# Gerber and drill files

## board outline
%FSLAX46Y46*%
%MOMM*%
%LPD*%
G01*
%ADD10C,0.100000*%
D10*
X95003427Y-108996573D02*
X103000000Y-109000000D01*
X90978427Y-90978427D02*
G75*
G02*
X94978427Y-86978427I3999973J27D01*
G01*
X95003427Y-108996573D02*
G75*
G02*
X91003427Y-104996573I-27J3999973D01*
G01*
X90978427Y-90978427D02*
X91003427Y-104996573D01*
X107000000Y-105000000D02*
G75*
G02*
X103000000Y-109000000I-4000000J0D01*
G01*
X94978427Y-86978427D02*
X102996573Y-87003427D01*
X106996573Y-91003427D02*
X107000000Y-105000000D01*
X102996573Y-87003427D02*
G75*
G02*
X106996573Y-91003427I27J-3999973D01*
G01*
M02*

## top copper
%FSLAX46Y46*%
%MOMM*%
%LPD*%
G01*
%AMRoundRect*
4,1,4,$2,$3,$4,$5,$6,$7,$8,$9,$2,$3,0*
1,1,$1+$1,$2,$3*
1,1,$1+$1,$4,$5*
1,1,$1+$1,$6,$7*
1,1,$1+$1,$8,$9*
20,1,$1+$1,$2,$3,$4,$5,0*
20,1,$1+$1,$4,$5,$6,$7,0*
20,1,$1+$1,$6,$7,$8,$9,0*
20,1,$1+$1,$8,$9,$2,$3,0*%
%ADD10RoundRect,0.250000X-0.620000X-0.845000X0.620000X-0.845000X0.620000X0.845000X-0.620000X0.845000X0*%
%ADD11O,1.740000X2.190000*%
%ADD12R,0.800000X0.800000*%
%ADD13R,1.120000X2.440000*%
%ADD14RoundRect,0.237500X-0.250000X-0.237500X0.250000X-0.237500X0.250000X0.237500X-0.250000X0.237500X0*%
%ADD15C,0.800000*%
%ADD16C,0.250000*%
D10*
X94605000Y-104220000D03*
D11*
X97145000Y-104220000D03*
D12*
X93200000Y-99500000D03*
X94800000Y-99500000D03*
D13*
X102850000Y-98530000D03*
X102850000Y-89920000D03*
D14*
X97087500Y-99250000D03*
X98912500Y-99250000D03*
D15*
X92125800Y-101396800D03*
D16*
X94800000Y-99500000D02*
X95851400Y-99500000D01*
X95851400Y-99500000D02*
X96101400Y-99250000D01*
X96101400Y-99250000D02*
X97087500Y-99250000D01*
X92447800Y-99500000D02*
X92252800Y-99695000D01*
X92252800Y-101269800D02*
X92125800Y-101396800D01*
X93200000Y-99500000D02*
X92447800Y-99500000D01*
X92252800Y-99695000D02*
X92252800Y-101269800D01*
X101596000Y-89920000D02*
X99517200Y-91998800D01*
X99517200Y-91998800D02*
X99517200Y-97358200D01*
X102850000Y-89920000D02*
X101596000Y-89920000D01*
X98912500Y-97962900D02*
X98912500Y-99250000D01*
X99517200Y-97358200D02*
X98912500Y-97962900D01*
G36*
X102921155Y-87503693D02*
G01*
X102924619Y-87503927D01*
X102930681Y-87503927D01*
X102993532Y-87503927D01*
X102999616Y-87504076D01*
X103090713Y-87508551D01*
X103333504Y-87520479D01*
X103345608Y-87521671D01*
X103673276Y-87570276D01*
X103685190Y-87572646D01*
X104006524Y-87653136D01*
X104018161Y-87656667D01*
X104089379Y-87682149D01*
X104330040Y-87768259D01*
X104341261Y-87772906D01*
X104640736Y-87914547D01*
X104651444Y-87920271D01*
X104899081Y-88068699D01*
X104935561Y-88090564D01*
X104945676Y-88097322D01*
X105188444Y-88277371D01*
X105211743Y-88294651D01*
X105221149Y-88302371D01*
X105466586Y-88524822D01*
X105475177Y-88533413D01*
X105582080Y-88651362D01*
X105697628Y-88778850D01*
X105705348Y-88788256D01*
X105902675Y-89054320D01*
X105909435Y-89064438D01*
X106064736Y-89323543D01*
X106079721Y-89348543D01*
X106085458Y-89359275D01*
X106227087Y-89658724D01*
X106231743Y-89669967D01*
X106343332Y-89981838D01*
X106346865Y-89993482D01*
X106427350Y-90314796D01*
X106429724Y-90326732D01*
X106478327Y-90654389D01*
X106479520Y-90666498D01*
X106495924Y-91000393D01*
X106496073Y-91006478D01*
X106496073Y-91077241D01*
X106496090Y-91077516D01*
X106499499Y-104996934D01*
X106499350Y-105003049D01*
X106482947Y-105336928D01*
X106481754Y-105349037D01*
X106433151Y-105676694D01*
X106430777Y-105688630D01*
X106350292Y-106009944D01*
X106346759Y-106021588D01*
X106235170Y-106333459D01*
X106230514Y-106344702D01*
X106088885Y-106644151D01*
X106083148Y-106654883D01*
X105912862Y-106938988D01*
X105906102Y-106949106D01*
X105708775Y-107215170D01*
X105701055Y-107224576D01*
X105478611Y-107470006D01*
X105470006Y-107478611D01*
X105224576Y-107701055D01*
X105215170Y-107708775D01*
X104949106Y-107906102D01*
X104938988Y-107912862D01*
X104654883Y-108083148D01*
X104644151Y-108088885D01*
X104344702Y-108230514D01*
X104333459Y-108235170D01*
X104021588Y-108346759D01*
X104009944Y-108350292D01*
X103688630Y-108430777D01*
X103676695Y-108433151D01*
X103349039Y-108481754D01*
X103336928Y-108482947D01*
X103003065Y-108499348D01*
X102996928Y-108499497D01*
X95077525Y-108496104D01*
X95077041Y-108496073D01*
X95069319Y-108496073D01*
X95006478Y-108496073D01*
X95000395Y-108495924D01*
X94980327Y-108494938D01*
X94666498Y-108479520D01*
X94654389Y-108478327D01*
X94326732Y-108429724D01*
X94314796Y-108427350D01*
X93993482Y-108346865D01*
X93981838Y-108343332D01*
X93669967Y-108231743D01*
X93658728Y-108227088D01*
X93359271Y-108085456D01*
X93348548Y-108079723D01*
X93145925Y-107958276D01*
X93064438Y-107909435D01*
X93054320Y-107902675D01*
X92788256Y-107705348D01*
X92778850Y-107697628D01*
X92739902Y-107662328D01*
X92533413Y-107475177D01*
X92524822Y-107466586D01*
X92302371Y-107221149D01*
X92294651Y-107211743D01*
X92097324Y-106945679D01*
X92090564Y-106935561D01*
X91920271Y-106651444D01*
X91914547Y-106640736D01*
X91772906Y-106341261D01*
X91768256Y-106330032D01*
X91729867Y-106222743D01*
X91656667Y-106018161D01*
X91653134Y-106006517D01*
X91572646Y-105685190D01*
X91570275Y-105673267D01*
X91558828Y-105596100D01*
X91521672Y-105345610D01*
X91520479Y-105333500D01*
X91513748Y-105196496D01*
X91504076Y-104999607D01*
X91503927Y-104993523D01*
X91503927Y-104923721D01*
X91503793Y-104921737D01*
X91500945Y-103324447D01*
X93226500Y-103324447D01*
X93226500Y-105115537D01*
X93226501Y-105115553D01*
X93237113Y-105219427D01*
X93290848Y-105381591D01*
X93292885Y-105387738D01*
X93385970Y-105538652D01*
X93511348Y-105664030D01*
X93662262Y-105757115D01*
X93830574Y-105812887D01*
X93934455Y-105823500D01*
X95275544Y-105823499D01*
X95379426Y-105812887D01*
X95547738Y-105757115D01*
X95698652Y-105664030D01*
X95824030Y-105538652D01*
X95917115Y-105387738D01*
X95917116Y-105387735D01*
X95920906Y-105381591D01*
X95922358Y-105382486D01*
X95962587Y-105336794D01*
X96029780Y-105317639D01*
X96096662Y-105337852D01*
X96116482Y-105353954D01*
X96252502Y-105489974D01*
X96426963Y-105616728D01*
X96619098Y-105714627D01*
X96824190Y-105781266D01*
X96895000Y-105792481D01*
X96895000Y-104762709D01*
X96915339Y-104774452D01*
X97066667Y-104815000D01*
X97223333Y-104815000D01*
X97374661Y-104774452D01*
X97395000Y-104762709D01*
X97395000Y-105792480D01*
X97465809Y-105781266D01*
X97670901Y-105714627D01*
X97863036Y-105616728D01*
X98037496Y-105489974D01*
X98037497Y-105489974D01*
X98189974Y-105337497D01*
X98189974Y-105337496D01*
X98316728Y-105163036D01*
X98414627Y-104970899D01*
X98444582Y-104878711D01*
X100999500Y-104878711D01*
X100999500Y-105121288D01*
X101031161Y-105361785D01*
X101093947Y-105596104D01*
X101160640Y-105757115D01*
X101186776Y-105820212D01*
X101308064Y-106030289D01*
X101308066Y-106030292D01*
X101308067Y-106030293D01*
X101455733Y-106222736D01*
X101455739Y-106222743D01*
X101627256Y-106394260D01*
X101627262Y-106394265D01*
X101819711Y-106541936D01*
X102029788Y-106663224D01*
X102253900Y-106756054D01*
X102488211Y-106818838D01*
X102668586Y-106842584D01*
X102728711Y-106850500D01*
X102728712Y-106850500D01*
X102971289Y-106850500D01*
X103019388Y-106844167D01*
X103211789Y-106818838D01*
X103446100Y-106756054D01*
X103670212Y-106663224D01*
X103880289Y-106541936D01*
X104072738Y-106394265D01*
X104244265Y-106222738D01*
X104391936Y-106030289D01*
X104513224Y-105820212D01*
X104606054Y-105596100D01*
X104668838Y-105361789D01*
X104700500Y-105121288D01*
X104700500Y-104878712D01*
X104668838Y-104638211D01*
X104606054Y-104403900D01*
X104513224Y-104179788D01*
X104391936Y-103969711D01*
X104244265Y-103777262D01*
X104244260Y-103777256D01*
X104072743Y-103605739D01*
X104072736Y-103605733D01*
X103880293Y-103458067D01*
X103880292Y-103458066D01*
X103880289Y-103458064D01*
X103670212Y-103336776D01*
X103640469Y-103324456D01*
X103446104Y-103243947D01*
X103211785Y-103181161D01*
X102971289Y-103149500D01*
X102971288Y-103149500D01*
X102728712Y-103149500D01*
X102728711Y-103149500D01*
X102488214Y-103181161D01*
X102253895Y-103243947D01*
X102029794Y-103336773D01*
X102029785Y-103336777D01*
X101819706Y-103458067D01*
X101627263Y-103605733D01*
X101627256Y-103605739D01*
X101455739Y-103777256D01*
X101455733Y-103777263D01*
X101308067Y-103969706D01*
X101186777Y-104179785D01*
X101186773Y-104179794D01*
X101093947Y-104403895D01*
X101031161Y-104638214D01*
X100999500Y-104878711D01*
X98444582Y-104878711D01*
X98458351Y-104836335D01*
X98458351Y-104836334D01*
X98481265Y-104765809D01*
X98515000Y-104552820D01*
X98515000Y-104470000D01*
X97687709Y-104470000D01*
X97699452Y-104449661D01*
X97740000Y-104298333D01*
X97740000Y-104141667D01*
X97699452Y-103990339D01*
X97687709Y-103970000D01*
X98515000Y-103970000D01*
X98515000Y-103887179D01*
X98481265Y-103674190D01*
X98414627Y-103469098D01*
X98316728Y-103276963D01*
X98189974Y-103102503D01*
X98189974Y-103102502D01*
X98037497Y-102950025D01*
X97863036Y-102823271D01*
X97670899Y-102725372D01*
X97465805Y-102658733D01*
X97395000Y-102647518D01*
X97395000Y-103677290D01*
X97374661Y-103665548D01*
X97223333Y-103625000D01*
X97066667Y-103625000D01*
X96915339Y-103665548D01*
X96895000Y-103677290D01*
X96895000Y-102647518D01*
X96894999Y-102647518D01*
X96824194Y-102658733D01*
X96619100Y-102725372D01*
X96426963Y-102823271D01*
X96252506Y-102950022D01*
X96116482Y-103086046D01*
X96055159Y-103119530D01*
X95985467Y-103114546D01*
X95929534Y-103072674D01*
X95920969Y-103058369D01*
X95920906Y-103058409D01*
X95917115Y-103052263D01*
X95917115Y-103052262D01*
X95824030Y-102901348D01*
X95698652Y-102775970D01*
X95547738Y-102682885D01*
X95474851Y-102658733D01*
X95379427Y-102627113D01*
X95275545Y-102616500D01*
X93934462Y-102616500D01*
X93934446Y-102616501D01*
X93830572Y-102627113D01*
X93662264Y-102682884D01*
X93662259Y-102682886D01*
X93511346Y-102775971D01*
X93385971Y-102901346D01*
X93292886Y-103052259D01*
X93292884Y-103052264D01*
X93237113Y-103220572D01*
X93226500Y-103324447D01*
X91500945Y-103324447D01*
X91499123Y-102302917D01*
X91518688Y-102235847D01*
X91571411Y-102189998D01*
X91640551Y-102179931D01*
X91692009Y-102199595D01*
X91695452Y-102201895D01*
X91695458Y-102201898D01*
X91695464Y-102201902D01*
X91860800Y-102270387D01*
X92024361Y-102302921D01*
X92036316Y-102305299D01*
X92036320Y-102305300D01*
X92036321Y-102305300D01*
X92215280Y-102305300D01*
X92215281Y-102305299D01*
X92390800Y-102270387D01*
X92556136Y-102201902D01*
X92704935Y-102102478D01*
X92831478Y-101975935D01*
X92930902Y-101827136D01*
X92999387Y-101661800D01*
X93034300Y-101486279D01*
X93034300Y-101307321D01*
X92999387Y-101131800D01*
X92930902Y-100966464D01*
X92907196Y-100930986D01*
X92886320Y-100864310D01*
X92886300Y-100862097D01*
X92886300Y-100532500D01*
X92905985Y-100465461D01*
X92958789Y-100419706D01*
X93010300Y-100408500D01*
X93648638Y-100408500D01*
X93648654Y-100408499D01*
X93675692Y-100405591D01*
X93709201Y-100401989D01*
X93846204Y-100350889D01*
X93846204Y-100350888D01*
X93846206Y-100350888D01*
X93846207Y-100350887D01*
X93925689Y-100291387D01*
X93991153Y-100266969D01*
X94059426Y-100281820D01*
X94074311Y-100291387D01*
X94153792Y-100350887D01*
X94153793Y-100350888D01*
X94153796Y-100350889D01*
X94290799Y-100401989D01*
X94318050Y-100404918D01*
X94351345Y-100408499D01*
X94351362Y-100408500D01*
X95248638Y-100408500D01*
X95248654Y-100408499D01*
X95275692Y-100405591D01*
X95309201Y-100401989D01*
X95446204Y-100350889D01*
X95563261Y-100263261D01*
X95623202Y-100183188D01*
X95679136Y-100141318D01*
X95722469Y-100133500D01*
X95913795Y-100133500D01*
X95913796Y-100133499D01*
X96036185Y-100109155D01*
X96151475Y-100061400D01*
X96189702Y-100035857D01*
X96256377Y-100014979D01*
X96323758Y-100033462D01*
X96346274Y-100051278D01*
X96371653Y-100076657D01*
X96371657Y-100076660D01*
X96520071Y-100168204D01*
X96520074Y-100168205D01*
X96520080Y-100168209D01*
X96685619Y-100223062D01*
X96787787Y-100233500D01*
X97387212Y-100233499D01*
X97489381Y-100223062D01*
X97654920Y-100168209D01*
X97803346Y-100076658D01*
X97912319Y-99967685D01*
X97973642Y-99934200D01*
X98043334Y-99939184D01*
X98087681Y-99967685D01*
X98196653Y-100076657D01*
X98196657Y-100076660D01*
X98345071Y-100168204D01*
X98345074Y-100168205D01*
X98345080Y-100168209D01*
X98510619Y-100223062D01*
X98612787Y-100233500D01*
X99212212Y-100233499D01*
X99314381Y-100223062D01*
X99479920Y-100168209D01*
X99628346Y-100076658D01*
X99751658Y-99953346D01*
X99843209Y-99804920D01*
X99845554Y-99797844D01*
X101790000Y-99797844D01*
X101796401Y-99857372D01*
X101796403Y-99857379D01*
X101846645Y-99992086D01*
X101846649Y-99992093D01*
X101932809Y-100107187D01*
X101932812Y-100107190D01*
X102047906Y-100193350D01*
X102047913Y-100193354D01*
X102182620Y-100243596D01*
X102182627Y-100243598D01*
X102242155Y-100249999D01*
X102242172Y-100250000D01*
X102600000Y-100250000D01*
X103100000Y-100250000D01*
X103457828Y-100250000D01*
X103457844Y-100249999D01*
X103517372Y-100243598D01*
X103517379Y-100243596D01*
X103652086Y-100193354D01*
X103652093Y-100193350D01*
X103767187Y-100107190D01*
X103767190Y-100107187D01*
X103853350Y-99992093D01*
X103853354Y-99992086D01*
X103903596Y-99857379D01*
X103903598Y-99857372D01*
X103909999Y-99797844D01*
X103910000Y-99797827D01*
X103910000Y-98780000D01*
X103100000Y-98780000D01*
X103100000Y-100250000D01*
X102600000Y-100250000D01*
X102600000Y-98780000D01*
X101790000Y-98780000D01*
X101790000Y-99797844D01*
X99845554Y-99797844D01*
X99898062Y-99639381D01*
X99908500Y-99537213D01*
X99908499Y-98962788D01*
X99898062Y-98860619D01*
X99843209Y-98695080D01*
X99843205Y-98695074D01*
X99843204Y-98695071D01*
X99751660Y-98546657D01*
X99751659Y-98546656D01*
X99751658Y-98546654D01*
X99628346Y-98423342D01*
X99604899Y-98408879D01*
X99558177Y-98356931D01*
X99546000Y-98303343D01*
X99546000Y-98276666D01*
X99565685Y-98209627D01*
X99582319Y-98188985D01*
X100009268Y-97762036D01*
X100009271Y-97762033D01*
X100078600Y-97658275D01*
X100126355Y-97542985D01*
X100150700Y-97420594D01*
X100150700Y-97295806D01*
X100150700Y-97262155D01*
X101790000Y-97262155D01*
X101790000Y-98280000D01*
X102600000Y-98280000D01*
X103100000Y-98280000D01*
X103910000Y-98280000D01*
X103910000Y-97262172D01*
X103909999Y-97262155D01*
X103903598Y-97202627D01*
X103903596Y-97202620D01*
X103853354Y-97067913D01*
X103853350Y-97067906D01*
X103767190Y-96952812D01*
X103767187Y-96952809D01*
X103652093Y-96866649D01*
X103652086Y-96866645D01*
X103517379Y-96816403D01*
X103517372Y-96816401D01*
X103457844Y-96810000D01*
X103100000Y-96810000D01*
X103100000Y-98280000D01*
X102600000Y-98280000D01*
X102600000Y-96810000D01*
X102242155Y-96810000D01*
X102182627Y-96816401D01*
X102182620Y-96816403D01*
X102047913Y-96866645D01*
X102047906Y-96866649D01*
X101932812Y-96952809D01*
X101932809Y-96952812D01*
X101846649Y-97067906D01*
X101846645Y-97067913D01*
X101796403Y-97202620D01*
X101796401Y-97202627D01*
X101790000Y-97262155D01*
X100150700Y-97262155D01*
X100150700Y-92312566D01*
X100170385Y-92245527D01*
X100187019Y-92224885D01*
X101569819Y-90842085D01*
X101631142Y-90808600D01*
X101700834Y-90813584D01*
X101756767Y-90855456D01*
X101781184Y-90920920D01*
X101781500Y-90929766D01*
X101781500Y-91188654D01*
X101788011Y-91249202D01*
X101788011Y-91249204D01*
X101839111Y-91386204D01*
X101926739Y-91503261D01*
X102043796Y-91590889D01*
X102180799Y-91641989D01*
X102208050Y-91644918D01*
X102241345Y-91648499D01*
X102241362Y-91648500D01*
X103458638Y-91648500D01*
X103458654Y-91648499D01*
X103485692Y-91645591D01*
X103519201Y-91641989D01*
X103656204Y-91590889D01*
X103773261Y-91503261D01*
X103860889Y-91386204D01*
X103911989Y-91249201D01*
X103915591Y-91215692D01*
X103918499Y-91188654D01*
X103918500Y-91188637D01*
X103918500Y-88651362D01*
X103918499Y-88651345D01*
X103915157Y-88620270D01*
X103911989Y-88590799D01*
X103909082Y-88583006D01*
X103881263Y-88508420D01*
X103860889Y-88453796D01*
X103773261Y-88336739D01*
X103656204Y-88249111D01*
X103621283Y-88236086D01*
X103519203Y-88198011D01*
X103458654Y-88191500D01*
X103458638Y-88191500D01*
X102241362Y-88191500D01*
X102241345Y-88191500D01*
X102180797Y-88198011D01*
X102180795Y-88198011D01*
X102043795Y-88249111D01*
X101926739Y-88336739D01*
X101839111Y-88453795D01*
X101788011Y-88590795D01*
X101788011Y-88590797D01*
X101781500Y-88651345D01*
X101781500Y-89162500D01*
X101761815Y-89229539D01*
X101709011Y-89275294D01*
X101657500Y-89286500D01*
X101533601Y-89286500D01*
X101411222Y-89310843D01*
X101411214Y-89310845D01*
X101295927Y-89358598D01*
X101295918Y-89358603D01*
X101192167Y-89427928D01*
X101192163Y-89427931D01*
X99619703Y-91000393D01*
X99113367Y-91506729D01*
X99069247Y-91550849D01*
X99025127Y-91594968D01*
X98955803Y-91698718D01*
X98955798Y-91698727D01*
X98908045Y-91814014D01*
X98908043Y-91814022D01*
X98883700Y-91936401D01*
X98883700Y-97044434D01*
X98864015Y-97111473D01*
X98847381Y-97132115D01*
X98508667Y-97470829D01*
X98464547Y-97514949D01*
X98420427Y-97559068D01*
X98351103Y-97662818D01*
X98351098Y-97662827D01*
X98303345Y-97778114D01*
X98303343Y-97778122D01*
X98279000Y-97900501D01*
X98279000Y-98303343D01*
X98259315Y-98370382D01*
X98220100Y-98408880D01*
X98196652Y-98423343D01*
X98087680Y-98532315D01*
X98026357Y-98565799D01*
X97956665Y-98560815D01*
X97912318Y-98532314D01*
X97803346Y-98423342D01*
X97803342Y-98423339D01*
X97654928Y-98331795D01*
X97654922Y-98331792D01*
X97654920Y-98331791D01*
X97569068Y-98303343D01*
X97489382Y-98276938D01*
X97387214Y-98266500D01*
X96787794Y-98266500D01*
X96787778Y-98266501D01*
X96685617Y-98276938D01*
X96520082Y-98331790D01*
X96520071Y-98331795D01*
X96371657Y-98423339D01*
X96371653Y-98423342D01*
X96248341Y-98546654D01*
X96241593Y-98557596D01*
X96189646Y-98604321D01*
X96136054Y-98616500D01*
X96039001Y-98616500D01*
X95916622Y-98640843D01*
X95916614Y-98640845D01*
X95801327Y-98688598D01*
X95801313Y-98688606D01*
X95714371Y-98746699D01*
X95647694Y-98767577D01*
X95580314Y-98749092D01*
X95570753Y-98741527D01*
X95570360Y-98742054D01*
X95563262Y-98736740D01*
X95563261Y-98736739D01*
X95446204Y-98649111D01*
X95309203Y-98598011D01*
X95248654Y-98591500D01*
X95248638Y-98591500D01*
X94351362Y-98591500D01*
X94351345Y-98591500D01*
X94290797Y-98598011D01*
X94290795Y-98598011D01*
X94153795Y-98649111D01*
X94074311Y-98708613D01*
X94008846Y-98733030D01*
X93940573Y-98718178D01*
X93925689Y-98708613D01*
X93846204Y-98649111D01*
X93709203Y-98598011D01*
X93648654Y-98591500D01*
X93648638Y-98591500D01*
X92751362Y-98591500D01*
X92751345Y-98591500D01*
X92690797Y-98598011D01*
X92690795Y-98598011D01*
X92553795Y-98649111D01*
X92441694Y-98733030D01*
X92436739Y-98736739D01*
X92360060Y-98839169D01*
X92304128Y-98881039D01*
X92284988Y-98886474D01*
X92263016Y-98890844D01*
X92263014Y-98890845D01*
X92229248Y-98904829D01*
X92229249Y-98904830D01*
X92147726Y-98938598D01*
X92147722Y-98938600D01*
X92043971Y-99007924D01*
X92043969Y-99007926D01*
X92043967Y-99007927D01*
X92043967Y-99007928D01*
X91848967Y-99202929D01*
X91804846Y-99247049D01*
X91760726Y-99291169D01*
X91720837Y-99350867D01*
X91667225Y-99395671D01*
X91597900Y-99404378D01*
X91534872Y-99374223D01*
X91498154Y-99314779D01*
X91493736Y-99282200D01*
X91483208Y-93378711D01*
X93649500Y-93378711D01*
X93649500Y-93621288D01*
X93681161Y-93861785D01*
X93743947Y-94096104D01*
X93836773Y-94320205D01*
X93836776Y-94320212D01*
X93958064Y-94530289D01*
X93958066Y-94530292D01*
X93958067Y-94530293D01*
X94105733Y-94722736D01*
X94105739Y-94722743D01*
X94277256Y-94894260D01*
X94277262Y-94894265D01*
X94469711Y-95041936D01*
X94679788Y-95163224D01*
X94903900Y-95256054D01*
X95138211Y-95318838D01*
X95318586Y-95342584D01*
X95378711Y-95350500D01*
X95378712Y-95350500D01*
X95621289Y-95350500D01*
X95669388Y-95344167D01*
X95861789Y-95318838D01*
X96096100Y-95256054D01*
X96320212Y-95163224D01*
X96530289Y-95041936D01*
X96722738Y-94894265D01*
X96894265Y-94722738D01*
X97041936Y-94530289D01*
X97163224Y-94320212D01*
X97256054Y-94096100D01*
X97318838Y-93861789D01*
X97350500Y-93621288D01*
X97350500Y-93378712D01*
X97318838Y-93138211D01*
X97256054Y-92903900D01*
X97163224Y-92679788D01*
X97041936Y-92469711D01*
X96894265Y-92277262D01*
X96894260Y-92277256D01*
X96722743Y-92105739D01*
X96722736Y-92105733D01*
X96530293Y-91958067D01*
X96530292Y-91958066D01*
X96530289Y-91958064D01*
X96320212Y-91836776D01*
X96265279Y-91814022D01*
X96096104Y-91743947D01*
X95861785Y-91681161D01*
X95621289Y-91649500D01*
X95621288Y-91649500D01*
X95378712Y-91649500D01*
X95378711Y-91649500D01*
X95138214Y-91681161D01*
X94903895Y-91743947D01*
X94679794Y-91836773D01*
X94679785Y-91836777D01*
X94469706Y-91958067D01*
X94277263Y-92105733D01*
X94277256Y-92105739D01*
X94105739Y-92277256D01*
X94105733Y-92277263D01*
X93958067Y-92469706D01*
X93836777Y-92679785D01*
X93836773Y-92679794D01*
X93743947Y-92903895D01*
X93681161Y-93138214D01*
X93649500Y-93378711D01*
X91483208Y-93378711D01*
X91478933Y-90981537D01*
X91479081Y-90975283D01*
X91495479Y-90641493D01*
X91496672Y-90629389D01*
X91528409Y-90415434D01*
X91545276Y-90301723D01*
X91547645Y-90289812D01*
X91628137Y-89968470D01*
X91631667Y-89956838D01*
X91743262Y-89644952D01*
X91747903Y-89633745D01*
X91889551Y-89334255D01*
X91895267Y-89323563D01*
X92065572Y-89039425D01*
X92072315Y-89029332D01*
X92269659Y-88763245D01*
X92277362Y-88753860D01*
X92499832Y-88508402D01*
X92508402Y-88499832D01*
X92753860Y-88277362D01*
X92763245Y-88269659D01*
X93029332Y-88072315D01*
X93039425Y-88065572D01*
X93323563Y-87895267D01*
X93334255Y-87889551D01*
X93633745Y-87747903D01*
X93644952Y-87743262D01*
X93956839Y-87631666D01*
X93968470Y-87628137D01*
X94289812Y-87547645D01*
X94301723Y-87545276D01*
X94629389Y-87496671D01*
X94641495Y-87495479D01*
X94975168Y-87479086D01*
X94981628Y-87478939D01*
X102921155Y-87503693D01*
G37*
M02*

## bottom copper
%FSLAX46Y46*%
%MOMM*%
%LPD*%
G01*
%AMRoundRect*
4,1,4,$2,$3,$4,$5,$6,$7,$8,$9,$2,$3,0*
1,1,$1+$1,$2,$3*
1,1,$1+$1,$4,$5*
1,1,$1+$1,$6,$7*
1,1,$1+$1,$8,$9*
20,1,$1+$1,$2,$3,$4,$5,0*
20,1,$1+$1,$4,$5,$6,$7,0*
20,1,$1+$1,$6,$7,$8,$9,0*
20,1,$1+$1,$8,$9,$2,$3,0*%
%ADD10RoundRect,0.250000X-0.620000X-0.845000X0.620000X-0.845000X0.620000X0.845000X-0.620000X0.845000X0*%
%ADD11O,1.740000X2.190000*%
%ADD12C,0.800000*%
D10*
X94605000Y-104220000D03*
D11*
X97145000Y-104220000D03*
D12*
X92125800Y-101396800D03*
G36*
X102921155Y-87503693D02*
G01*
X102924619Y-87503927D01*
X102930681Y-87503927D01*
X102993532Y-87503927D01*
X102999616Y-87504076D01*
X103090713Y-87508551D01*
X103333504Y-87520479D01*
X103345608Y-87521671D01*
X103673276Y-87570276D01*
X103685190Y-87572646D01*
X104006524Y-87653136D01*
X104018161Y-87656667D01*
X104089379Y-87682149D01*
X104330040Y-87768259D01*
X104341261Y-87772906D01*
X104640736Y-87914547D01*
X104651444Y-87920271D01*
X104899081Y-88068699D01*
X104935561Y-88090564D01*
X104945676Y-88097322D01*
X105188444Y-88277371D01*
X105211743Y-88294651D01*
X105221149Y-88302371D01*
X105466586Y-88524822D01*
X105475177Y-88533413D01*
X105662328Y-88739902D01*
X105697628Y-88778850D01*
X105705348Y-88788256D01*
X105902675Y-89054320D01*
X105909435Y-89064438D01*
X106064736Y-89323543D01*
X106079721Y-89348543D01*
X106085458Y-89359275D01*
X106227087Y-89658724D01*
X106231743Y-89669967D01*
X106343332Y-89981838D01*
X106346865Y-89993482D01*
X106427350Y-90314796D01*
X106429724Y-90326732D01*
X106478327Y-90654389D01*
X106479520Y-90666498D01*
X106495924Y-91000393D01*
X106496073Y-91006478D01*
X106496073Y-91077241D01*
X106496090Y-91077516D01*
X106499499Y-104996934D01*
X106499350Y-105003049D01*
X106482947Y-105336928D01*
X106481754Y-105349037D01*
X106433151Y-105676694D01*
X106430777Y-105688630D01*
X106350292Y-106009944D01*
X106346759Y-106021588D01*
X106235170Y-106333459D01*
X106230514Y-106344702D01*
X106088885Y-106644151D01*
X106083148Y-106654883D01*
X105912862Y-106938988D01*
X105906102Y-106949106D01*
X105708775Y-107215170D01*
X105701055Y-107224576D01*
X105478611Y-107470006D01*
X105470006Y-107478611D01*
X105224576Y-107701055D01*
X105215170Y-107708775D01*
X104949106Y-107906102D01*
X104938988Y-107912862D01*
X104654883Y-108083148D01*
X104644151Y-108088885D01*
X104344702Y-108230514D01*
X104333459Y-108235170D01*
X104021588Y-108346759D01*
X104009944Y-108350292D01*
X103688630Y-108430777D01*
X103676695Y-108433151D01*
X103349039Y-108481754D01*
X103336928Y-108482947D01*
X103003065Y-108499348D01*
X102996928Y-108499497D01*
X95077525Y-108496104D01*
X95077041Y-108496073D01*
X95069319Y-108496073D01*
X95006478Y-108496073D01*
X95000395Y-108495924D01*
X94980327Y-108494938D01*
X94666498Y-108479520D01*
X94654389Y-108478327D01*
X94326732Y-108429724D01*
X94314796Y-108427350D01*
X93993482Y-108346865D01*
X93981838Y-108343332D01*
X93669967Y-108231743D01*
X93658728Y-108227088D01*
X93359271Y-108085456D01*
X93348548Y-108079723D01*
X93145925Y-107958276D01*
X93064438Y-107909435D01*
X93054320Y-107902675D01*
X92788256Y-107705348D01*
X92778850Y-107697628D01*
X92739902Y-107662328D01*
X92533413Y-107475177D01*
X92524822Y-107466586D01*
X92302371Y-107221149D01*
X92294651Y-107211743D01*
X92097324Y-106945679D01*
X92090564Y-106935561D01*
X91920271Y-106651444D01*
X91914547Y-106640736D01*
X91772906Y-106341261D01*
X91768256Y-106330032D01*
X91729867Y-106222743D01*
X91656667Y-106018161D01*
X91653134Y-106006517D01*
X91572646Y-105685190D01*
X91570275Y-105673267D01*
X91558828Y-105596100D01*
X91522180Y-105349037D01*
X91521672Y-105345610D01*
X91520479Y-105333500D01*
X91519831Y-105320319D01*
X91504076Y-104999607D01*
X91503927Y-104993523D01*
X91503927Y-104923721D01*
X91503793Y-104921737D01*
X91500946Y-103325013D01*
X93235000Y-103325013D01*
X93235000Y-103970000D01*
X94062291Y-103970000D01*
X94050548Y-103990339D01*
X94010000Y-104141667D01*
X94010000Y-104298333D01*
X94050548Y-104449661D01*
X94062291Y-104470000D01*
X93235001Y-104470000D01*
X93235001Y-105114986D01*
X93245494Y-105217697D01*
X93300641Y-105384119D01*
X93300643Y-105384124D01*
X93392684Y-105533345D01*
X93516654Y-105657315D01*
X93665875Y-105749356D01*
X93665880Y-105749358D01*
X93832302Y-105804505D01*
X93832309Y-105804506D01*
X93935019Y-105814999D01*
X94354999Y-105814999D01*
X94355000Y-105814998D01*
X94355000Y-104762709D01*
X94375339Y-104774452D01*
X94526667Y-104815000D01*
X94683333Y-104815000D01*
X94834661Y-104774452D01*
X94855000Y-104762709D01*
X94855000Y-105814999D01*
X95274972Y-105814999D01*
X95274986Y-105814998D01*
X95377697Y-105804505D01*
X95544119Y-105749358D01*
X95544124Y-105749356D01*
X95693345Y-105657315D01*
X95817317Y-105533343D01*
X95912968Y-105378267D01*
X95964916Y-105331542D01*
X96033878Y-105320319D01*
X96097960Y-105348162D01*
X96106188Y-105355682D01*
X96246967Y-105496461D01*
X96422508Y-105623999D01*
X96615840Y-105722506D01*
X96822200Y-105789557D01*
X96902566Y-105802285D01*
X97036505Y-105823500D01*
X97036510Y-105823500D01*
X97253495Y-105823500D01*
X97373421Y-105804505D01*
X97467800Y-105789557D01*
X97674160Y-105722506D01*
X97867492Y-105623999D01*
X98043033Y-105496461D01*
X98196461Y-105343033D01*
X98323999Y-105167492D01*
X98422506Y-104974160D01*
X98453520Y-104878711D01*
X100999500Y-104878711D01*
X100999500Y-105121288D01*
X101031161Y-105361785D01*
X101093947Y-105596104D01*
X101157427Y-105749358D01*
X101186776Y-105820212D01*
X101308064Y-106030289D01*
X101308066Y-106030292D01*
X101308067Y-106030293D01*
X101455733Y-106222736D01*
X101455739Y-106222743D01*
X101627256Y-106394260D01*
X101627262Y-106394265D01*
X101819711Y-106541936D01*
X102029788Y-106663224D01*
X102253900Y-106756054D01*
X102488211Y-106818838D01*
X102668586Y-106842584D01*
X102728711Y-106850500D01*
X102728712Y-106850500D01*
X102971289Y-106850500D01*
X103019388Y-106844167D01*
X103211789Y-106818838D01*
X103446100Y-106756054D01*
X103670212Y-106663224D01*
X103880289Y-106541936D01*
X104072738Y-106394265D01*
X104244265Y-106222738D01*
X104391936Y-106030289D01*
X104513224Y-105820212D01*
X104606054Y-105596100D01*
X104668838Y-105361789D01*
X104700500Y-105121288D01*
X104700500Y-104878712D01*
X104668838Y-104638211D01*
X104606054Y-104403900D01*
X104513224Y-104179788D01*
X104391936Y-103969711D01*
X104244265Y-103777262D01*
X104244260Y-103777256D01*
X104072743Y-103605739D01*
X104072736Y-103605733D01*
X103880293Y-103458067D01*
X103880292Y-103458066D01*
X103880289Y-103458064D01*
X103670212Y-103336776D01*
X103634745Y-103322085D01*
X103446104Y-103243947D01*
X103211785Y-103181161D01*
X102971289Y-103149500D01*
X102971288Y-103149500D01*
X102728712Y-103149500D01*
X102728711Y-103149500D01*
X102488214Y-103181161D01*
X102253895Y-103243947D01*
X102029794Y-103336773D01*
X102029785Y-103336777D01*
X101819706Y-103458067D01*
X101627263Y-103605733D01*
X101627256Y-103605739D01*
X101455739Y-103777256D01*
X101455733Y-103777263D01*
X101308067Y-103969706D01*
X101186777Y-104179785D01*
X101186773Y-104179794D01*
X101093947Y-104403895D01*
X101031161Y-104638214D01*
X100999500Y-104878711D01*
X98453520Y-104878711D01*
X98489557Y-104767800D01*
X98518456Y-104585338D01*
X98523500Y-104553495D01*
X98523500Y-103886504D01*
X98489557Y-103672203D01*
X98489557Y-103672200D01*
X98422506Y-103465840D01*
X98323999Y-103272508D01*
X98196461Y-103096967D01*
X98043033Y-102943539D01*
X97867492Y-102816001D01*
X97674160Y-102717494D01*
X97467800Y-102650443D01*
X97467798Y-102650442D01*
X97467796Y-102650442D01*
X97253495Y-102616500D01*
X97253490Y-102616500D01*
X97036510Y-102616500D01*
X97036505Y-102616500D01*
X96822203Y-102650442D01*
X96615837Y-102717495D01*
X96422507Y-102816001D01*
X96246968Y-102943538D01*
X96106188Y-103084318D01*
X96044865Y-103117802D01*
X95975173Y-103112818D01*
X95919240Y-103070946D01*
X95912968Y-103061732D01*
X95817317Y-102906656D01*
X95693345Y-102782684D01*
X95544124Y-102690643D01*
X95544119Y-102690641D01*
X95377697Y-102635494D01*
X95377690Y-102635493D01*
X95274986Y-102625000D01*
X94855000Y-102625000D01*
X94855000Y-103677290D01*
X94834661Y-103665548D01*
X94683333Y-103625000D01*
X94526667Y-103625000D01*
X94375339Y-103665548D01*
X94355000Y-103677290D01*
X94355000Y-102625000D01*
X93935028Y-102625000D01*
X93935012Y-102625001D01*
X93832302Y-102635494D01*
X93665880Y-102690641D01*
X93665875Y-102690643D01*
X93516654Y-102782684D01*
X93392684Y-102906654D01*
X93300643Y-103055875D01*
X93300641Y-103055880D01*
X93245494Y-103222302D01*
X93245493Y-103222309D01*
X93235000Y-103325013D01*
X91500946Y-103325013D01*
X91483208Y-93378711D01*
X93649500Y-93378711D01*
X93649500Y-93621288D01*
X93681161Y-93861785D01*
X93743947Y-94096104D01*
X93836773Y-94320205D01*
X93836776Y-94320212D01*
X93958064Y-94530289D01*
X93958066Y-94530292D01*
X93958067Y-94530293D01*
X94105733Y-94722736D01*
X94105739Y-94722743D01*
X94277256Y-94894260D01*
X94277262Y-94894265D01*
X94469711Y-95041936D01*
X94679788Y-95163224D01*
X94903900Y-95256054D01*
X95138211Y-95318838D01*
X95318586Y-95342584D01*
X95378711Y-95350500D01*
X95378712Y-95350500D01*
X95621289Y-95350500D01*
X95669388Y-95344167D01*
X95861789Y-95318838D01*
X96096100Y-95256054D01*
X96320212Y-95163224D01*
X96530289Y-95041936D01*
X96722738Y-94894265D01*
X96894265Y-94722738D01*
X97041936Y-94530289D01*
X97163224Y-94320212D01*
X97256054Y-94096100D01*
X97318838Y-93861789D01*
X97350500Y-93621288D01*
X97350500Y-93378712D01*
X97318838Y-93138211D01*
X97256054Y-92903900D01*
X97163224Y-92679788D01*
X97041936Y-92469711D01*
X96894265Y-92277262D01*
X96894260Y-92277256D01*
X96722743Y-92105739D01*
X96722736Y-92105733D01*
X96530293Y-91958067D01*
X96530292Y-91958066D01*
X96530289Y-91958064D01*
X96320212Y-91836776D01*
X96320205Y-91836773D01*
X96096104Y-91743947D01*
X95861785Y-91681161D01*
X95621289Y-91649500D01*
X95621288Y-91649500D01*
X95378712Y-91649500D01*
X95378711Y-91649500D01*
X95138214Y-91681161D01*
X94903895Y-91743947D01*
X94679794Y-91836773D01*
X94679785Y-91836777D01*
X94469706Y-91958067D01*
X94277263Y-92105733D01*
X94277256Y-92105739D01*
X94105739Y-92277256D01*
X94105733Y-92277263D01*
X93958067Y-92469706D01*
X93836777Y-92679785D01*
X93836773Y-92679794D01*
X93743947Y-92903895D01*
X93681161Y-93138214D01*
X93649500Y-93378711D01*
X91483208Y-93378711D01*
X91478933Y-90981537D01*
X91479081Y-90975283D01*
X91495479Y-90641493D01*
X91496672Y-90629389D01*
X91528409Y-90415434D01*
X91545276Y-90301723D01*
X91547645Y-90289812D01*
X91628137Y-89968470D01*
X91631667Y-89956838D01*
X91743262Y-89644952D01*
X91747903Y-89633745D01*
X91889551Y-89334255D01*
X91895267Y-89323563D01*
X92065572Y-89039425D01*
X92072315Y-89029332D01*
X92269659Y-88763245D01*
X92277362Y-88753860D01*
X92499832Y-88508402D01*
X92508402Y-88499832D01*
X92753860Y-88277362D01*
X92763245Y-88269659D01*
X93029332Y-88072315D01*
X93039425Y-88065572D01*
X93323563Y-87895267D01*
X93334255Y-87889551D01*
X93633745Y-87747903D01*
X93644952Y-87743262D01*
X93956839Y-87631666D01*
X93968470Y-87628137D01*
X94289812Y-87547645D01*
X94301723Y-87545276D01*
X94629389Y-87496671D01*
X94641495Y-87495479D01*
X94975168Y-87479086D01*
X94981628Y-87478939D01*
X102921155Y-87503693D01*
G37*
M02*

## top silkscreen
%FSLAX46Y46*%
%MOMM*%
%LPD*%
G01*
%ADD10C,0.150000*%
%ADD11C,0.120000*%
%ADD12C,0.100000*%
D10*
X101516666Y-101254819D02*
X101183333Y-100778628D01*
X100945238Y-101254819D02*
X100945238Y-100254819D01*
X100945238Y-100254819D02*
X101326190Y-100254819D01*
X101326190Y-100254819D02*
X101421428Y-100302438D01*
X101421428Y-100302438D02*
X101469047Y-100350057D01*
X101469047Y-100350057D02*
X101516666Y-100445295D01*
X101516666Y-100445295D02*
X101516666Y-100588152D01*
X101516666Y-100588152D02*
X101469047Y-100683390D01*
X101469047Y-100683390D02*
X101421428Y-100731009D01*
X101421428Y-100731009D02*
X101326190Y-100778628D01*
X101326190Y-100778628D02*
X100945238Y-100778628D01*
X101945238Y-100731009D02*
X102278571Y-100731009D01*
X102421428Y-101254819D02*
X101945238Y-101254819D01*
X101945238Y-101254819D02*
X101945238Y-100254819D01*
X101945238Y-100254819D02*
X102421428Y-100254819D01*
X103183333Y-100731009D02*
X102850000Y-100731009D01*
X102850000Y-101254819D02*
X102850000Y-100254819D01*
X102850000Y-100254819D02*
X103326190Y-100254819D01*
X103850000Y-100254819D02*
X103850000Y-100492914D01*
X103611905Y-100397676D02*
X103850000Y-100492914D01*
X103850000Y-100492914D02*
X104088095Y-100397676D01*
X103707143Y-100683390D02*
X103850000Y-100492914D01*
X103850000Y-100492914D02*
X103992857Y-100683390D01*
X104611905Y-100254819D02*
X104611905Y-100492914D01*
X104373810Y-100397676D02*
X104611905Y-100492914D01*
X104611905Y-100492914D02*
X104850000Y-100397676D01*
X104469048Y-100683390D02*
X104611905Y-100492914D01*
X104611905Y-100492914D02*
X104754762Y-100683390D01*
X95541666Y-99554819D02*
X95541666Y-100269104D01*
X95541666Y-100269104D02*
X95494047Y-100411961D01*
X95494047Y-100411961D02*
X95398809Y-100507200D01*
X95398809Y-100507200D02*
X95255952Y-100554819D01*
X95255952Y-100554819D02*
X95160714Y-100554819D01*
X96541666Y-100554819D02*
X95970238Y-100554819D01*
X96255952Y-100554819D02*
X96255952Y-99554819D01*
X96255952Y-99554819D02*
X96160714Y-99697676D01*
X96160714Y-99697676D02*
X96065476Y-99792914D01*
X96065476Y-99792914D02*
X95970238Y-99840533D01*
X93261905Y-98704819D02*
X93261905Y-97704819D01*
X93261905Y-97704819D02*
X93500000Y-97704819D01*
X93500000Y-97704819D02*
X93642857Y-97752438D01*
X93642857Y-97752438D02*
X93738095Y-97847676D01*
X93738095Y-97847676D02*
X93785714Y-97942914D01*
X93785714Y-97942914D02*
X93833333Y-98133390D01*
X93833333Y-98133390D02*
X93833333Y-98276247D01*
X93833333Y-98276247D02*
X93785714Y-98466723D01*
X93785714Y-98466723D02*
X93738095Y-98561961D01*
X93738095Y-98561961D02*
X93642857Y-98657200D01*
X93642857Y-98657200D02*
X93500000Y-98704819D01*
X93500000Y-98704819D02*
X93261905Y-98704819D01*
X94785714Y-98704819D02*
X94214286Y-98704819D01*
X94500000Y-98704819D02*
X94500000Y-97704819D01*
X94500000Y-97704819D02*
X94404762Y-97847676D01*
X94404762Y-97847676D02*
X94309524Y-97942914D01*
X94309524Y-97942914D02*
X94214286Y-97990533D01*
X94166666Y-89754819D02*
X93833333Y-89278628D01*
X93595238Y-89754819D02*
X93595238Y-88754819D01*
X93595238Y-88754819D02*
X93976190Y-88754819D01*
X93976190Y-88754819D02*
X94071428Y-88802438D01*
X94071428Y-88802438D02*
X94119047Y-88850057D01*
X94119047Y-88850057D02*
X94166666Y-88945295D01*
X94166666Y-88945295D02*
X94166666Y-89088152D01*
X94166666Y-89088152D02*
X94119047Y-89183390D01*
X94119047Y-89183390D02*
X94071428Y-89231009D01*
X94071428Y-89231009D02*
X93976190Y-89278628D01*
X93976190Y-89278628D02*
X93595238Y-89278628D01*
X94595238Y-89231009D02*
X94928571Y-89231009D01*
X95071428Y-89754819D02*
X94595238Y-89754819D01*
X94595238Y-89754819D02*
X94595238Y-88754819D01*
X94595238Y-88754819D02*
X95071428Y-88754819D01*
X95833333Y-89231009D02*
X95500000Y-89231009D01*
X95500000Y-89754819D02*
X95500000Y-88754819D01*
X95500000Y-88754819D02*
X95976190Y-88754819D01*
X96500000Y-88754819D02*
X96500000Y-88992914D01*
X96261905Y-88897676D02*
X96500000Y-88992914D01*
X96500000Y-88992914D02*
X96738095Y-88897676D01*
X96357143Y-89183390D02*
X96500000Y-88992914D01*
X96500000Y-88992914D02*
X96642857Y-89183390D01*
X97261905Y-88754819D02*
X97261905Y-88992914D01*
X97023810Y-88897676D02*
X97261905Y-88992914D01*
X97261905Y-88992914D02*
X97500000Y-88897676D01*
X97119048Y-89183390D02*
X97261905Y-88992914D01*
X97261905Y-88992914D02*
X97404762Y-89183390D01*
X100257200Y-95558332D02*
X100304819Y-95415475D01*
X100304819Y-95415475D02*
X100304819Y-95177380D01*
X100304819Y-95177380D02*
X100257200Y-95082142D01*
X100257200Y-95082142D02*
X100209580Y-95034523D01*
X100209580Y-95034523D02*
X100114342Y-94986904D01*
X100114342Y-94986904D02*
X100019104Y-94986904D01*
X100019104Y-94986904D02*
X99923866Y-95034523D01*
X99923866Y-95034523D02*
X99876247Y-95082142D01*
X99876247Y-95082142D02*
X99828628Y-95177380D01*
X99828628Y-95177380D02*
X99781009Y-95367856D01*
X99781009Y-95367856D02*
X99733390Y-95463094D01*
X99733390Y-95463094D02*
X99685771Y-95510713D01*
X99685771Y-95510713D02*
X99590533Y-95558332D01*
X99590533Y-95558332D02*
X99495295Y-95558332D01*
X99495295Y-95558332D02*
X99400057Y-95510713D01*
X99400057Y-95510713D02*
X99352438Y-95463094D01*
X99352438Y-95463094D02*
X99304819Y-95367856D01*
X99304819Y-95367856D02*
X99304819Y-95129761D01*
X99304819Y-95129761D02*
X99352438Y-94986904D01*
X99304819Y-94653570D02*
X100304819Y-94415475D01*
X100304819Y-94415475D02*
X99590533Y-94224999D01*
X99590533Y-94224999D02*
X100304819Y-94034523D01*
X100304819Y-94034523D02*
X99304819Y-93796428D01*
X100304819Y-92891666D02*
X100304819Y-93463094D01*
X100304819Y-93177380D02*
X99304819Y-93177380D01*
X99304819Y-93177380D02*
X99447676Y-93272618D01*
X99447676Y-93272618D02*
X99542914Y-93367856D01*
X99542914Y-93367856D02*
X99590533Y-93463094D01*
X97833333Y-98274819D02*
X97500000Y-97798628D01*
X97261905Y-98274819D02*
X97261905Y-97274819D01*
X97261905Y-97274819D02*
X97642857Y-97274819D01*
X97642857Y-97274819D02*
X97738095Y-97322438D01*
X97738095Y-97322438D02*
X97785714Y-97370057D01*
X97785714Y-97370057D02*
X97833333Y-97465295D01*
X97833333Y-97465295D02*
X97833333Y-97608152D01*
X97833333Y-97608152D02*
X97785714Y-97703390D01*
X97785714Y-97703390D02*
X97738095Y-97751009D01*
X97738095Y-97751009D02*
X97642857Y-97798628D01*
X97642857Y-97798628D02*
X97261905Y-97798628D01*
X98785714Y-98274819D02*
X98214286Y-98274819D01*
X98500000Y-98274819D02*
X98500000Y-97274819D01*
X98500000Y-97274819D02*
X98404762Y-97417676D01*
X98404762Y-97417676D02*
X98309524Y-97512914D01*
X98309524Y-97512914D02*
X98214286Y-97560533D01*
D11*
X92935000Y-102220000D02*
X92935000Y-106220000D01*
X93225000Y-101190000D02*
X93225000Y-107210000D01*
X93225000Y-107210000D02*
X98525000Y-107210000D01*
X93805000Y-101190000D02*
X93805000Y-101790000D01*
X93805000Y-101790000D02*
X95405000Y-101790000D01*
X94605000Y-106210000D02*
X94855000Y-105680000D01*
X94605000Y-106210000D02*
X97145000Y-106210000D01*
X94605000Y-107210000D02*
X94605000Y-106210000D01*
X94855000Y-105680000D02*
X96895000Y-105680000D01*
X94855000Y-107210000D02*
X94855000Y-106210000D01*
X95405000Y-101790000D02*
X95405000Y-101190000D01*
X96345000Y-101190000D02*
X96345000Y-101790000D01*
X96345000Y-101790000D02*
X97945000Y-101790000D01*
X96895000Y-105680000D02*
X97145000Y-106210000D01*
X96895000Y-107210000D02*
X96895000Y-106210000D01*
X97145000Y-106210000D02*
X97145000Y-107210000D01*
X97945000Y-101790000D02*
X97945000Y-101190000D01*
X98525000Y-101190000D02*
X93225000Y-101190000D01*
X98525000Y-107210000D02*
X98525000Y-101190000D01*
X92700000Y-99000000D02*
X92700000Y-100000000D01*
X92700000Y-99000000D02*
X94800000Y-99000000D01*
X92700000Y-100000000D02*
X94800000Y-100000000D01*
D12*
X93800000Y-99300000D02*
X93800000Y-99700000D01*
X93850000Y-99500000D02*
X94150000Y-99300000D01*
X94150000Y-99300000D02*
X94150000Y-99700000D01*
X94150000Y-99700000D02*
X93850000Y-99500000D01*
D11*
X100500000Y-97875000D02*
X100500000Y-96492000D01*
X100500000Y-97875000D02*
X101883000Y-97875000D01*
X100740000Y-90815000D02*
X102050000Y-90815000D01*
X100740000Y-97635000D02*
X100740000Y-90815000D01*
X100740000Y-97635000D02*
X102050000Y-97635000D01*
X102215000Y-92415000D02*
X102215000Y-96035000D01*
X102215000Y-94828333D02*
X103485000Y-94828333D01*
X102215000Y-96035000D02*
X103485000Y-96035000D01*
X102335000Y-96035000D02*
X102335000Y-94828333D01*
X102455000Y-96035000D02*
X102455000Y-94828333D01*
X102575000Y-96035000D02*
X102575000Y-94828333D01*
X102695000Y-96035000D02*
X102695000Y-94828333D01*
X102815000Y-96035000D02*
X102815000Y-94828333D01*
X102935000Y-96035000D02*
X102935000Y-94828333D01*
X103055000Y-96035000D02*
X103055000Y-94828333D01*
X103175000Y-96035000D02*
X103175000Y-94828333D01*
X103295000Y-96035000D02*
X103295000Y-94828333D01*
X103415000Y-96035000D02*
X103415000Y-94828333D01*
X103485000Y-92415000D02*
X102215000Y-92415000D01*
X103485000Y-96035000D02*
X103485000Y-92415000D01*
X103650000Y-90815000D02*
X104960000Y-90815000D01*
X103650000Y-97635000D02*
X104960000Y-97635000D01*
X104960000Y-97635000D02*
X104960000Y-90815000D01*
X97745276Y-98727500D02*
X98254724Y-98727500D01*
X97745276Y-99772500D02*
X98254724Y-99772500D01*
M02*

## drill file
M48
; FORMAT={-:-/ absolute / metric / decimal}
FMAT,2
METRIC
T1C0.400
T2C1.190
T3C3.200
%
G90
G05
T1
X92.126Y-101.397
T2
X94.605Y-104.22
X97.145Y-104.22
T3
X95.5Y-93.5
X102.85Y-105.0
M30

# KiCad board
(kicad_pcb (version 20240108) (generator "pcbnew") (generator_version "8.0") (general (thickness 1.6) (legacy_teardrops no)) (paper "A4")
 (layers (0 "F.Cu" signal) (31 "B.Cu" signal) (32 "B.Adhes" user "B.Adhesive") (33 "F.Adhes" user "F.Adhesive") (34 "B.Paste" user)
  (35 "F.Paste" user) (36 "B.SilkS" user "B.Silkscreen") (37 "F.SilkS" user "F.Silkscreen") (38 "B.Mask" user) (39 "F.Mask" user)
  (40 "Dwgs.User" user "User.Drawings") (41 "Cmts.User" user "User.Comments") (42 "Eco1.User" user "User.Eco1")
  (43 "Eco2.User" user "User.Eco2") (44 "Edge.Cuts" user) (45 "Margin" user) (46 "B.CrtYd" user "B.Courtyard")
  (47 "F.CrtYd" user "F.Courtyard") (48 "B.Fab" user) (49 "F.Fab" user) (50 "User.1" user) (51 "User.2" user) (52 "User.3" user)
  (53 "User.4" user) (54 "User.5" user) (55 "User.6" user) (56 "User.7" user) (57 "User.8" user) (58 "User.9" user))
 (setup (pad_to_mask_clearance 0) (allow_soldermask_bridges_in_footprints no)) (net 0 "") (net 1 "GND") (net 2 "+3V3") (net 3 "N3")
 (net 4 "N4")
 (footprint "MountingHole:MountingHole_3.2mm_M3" (layer "F.Cu") (at 102.85 105)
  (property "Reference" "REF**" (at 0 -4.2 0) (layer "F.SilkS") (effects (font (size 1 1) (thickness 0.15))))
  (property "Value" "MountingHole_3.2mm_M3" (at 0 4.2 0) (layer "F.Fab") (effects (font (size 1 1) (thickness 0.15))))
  (pad "" np_thru_hole circle (at 0 0) (size 3.2 3.2) (drill 3.2) (layers "*.Cu" "*.Mask")))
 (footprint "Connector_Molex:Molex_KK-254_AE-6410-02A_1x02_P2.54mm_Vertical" (layer "F.Cu") (at 94.605 104.22)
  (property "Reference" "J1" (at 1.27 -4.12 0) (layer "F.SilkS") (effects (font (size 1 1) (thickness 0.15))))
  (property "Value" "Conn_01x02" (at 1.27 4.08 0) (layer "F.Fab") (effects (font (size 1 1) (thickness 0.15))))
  (fp_line (start -1.67 -2) (end -1.67 2) (stroke (width 0.12) (type solid)) (layer "F.SilkS"))
  (fp_line (start -1.38 -3.03) (end -1.38 2.99) (stroke (width 0.12) (type solid)) (layer "F.SilkS"))
  (fp_line (start -1.38 2.99) (end 3.92 2.99) (stroke (width 0.12) (type solid)) (layer "F.SilkS"))
  (fp_line (start -0.8 -3.03) (end -0.8 -2.43) (stroke (width 0.12) (type solid)) (layer "F.SilkS"))
  (fp_line (start -0.8 -2.43) (end 0.8 -2.43) (stroke (width 0.12) (type solid)) (layer "F.SilkS"))
  (fp_line (start 0 1.99) (end 0.25 1.46) (stroke (width 0.12) (type solid)) (layer "F.SilkS"))
  (fp_line (start 0 1.99) (end 2.54 1.99) (stroke (width 0.12) (type solid)) (layer "F.SilkS"))
  (fp_line (start 0 2.99) (end 0 1.99) (stroke (width 0.12) (type solid)) (layer "F.SilkS"))
  (fp_line (start 0.25 1.46) (end 2.29 1.46) (stroke (width 0.12) (type solid)) (layer "F.SilkS"))
  (fp_line (start 0.25 2.99) (end 0.25 1.99) (stroke (width 0.12) (type solid)) (layer "F.SilkS"))
  (fp_line (start 0.8 -2.43) (end 0.8 -3.03) (stroke (width 0.12) (type solid)) (layer "F.SilkS"))
  (fp_line (start 1.74 -3.03) (end 1.74 -2.43) (stroke (width 0.12) (type solid)) (layer "F.SilkS"))
  (fp_line (start 1.74 -2.43) (end 3.34 -2.43) (stroke (width 0.12) (type solid)) (layer "F.SilkS"))
  (fp_line (start 2.29 1.46) (end 2.54 1.99) (stroke (width 0.12) (type solid)) (layer "F.SilkS"))
  (fp_line (start 2.29 2.99) (end 2.29 1.99) (stroke (width 0.12) (type solid)) (layer "F.SilkS"))
  (fp_line (start 2.54 1.99) (end 2.54 2.99) (stroke (width 0.12) (type solid)) (layer "F.SilkS"))
  (fp_line (start 3.34 -2.43) (end 3.34 -3.03) (stroke (width 0.12) (type solid)) (layer "F.SilkS"))
  (fp_line (start 3.92 -3.03) (end -1.38 -3.03) (stroke (width 0.12) (type solid)) (layer "F.SilkS"))
  (fp_line (start 3.92 2.99) (end 3.92 -3.03) (stroke (width 0.12) (type solid)) (layer "F.SilkS"))
  (pad "1" thru_hole roundrect (at 0 0) (size 1.74 2.19) (drill 1.19) (layers "*.Cu" "*.Mask") (remove_unused_layers no)
   (roundrect_rratio 0.143678) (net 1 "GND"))
  (pad "2" thru_hole oval (at 2.54 0) (size 1.74 2.19) (drill 1.19) (layers "*.Cu" "*.Mask") (remove_unused_layers no) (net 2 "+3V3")))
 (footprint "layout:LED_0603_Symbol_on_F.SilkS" (layer "F.Cu") (at 94 99.5)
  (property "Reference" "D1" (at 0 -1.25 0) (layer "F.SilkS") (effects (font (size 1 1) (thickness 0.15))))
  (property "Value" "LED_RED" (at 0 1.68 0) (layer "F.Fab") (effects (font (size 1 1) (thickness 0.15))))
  (fp_line (start -1.3 -0.5) (end -1.3 0.5) (stroke (width 0.12) (type solid)) (layer "F.SilkS"))
  (fp_line (start -1.3 -0.5) (end 0.8 -0.5) (stroke (width 0.12) (type solid)) (layer "F.SilkS"))
  (fp_line (start -1.3 0.5) (end 0.8 0.5) (stroke (width 0.12) (type solid)) (layer "F.SilkS"))
  (fp_line (start -0.2 -0.2) (end -0.2 0.2) (stroke (width 0.1) (type solid)) (layer "F.SilkS"))
  (fp_line (start -0.15 0) (end 0.15 -0.2) (stroke (width 0.1) (type solid)) (layer "F.SilkS"))
  (fp_line (start 0.15 -0.2) (end 0.15 0.2) (stroke (width 0.1) (type solid)) (layer "F.SilkS"))
  (fp_line (start 0.15 0.2) (end -0.15 0) (stroke (width 0.1) (type solid)) (layer "F.SilkS"))
  (pad "1" smd rect (at -0.8 0 180) (size 0.8 0.8) (layers "F.Cu" "F.Paste" "F.Mask") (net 1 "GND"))
  (pad "2" smd rect (at 0.8 0 180) (size 0.8 0.8) (layers "F.Cu" "F.Paste" "F.Mask") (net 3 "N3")))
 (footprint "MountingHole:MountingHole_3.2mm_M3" (layer "F.Cu") (at 95.5 93.5)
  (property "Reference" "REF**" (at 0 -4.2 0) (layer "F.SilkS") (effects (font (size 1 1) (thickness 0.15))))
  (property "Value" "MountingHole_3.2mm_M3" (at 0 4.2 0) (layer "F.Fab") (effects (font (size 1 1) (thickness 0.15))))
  (pad "" np_thru_hole circle (at 0 0) (size 3.2 3.2) (drill 3.2) (layers "*.Cu" "*.Mask")))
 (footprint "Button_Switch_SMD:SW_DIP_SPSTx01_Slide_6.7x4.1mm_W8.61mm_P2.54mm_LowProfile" (layer "F.Cu") (at 102.85 94.225 90)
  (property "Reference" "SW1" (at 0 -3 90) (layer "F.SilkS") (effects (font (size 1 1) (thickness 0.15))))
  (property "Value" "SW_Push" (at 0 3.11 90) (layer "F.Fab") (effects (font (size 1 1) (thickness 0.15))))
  (fp_line (start -3.65 -2.35) (end -2.267 -2.35) (stroke (width 0.12) (type solid)) (layer "F.SilkS"))
  (fp_line (start -3.65 -2.35) (end -3.65 -0.967) (stroke (width 0.12) (type solid)) (layer "F.SilkS"))
  (fp_line (start 3.41 -2.11) (end 3.41 -0.8) (stroke (width 0.12) (type solid)) (layer "F.SilkS"))
  (fp_line (start -3.41 -2.11) (end 3.41 -2.11) (stroke (width 0.12) (type solid)) (layer "F.SilkS"))
  (fp_line (start -3.41 -2.11) (end -3.41 -0.8) (stroke (width 0.12) (type solid)) (layer "F.SilkS"))
  (fp_line (start 1.81 -0.635) (end -1.81 -0.635) (stroke (width 0.12) (type solid)) (layer "F.SilkS"))
  (fp_line (start -0.603333 -0.635) (end -0.603333 0.635) (stroke (width 0.12) (type solid)) (layer "F.SilkS"))
  (fp_line (start -1.81 -0.635) (end -1.81 0.635) (stroke (width 0.12) (type solid)) (layer "F.SilkS"))
  (fp_line (start -1.81 -0.515) (end -0.603333 -0.515) (stroke (width 0.12) (type solid)) (layer "F.SilkS"))
  (fp_line (start -1.81 -0.395) (end -0.603333 -0.395) (stroke (width 0.12) (type solid)) (layer "F.SilkS"))
  (fp_line (start -1.81 -0.275) (end -0.603333 -0.275) (stroke (width 0.12) (type solid)) (layer "F.SilkS"))
  (fp_line (start -1.81 -0.155) (end -0.603333 -0.155) (stroke (width 0.12) (type solid)) (layer "F.SilkS"))
  (fp_line (start -1.81 -0.035) (end -0.603333 -0.035) (stroke (width 0.12) (type solid)) (layer "F.SilkS"))
  (fp_line (start -1.81 0.085) (end -0.603333 0.085) (stroke (width 0.12) (type solid)) (layer "F.SilkS"))
  (fp_line (start -1.81 0.205) (end -0.603333 0.205) (stroke (width 0.12) (type solid)) (layer "F.SilkS"))
  (fp_line (start -1.81 0.325) (end -0.603333 0.325) (stroke (width 0.12) (type solid)) (layer "F.SilkS"))
  (fp_line (start -1.81 0.445) (end -0.603333 0.445) (stroke (width 0.12) (type solid)) (layer "F.SilkS"))
  (fp_line (start -1.81 0.565) (end -0.603333 0.565) (stroke (width 0.12) (type solid)) (layer "F.SilkS"))
  (fp_line (start 1.81 0.635) (end 1.81 -0.635) (stroke (width 0.12) (type solid)) (layer "F.SilkS"))
  (fp_line (start -1.81 0.635) (end 1.81 0.635) (stroke (width 0.12) (type solid)) (layer "F.SilkS"))
  (fp_line (start 3.41 0.8) (end 3.41 2.11) (stroke (width 0.12) (type solid)) (layer "F.SilkS"))
  (fp_line (start -3.41 0.8) (end -3.41 2.11) (stroke (width 0.12) (type solid)) (layer "F.SilkS"))
  (fp_line (start -3.41 2.11) (end 3.41 2.11) (stroke (width 0.12) (type solid)) (layer "F.SilkS"))
  (pad "1" smd rect (at -4.305 0 90) (size 2.44 1.12) (layers "F.Cu" "F.Paste" "F.Mask") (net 2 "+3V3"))
  (pad "2" smd rect (at 4.305 0 90) (size 2.44 1.12) (layers "F.Cu" "F.Paste" "F.Mask") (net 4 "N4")))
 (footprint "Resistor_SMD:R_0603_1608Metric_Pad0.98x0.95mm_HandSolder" (layer "F.Cu") (at 98 99.25)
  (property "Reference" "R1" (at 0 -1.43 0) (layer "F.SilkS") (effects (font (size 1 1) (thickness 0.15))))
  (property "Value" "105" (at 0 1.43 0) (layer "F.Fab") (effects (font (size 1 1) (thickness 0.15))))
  (fp_line (start -0.254724 -0.5225) (end 0.254724 -0.5225) (stroke (width 0.12) (type solid)) (layer "F.SilkS"))
  (fp_line (start -0.254724 0.5225) (end 0.254724 0.5225) (stroke (width 0.12) (type solid)) (layer "F.SilkS"))
  (pad "1" smd roundrect (at -0.9125 0) (size 0.975 0.95) (layers "F.Cu" "F.Paste" "F.Mask") (roundrect_rratio 0.25) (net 3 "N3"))
  (pad "2" smd roundrect (at 0.9125 0) (size 0.975 0.95) (layers "F.Cu" "F.Paste" "F.Mask") (roundrect_rratio 0.25) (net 4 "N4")))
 (gr_line (start 95.003427 108.996573) (end 103 109) (stroke (width 0.1) (type default)) (layer "Edge.Cuts"))
 (gr_arc (start 90.978427 90.978427) (mid 92.15 88.15) (end 94.978427 86.978427) (stroke (width 0.1) (type default)) (layer "Edge.Cuts"))
 (gr_arc (start 95.003427 108.996573) (mid 92.175 107.825) (end 91.003427 104.996573) (stroke (width 0.1) (type default))
  (layer "Edge.Cuts"))
 (gr_line (start 90.978427 90.978427) (end 91.003427 104.996573) (stroke (width 0.1) (type default)) (layer "Edge.Cuts"))
 (gr_arc (start 107 105) (mid 105.828427 107.828427) (end 103 109) (stroke (width 0.1) (type default)) (layer "Edge.Cuts"))
 (gr_line (start 94.978427 86.978427) (end 102.996573 87.003427) (stroke (width 0.1) (type default)) (layer "Edge.Cuts"))
 (gr_line (start 106.996573 91.003427) (end 107 105) (stroke (width 0.1) (type default)) (layer "Edge.Cuts"))
 (gr_arc (start 102.996573 87.003427) (mid 105.825 88.175) (end 106.996573 91.003427) (stroke (width 0.1) (type default))
  (layer "Edge.Cuts"))
 (segment (start 94.8 99.5) (end 95.8514 99.5) (width 0.25) (layer "F.Cu") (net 3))
 (segment (start 95.8514 99.5) (end 96.1014 99.25) (width 0.25) (layer "F.Cu") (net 3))
 (segment (start 96.1014 99.25) (end 97.0875 99.25) (width 0.25) (layer "F.Cu") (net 3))
 (segment (start 92.4478 99.5) (end 92.2528 99.695) (width 0.25) (layer "F.Cu") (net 1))
 (segment (start 92.2528 101.2698) (end 92.1258 101.3968) (width 0.25) (layer "F.Cu") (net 1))
 (segment (start 93.2 99.5) (end 92.4478 99.5) (width 0.25) (layer "F.Cu") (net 1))
 (segment (start 92.2528 99.695) (end 92.2528 101.2698) (width 0.25) (layer "F.Cu") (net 1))
 (via (at 92.1258 101.3968) (size 0.8) (drill 0.4) (layers "F.Cu" "B.Cu") (free yes) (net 1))
 (segment (start 101.596 89.92) (end 99.5172 91.9988) (width 0.25) (layer "F.Cu") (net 4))
 (segment (start 99.5172 91.9988) (end 99.5172 97.3582) (width 0.25) (layer "F.Cu") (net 4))
 (segment (start 102.85 89.92) (end 101.596 89.92) (width 0.25) (layer "F.Cu") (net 4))
 (segment (start 98.9125 97.9629) (end 98.9125 99.25) (width 0.25) (layer "F.Cu") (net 4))
 (segment (start 99.5172 97.3582) (end 98.9125 97.9629) (width 0.25) (layer "F.Cu") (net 4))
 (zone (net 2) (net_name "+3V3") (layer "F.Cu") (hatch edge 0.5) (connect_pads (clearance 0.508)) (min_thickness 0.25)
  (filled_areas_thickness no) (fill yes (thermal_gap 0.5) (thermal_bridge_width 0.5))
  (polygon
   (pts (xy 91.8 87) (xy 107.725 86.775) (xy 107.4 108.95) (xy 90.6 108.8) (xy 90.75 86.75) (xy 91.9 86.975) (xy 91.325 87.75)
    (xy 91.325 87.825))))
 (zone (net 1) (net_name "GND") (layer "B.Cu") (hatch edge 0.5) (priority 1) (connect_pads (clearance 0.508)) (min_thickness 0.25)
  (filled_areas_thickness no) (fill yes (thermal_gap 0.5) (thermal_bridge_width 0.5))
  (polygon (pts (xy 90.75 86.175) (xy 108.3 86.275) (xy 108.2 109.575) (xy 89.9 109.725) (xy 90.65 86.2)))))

